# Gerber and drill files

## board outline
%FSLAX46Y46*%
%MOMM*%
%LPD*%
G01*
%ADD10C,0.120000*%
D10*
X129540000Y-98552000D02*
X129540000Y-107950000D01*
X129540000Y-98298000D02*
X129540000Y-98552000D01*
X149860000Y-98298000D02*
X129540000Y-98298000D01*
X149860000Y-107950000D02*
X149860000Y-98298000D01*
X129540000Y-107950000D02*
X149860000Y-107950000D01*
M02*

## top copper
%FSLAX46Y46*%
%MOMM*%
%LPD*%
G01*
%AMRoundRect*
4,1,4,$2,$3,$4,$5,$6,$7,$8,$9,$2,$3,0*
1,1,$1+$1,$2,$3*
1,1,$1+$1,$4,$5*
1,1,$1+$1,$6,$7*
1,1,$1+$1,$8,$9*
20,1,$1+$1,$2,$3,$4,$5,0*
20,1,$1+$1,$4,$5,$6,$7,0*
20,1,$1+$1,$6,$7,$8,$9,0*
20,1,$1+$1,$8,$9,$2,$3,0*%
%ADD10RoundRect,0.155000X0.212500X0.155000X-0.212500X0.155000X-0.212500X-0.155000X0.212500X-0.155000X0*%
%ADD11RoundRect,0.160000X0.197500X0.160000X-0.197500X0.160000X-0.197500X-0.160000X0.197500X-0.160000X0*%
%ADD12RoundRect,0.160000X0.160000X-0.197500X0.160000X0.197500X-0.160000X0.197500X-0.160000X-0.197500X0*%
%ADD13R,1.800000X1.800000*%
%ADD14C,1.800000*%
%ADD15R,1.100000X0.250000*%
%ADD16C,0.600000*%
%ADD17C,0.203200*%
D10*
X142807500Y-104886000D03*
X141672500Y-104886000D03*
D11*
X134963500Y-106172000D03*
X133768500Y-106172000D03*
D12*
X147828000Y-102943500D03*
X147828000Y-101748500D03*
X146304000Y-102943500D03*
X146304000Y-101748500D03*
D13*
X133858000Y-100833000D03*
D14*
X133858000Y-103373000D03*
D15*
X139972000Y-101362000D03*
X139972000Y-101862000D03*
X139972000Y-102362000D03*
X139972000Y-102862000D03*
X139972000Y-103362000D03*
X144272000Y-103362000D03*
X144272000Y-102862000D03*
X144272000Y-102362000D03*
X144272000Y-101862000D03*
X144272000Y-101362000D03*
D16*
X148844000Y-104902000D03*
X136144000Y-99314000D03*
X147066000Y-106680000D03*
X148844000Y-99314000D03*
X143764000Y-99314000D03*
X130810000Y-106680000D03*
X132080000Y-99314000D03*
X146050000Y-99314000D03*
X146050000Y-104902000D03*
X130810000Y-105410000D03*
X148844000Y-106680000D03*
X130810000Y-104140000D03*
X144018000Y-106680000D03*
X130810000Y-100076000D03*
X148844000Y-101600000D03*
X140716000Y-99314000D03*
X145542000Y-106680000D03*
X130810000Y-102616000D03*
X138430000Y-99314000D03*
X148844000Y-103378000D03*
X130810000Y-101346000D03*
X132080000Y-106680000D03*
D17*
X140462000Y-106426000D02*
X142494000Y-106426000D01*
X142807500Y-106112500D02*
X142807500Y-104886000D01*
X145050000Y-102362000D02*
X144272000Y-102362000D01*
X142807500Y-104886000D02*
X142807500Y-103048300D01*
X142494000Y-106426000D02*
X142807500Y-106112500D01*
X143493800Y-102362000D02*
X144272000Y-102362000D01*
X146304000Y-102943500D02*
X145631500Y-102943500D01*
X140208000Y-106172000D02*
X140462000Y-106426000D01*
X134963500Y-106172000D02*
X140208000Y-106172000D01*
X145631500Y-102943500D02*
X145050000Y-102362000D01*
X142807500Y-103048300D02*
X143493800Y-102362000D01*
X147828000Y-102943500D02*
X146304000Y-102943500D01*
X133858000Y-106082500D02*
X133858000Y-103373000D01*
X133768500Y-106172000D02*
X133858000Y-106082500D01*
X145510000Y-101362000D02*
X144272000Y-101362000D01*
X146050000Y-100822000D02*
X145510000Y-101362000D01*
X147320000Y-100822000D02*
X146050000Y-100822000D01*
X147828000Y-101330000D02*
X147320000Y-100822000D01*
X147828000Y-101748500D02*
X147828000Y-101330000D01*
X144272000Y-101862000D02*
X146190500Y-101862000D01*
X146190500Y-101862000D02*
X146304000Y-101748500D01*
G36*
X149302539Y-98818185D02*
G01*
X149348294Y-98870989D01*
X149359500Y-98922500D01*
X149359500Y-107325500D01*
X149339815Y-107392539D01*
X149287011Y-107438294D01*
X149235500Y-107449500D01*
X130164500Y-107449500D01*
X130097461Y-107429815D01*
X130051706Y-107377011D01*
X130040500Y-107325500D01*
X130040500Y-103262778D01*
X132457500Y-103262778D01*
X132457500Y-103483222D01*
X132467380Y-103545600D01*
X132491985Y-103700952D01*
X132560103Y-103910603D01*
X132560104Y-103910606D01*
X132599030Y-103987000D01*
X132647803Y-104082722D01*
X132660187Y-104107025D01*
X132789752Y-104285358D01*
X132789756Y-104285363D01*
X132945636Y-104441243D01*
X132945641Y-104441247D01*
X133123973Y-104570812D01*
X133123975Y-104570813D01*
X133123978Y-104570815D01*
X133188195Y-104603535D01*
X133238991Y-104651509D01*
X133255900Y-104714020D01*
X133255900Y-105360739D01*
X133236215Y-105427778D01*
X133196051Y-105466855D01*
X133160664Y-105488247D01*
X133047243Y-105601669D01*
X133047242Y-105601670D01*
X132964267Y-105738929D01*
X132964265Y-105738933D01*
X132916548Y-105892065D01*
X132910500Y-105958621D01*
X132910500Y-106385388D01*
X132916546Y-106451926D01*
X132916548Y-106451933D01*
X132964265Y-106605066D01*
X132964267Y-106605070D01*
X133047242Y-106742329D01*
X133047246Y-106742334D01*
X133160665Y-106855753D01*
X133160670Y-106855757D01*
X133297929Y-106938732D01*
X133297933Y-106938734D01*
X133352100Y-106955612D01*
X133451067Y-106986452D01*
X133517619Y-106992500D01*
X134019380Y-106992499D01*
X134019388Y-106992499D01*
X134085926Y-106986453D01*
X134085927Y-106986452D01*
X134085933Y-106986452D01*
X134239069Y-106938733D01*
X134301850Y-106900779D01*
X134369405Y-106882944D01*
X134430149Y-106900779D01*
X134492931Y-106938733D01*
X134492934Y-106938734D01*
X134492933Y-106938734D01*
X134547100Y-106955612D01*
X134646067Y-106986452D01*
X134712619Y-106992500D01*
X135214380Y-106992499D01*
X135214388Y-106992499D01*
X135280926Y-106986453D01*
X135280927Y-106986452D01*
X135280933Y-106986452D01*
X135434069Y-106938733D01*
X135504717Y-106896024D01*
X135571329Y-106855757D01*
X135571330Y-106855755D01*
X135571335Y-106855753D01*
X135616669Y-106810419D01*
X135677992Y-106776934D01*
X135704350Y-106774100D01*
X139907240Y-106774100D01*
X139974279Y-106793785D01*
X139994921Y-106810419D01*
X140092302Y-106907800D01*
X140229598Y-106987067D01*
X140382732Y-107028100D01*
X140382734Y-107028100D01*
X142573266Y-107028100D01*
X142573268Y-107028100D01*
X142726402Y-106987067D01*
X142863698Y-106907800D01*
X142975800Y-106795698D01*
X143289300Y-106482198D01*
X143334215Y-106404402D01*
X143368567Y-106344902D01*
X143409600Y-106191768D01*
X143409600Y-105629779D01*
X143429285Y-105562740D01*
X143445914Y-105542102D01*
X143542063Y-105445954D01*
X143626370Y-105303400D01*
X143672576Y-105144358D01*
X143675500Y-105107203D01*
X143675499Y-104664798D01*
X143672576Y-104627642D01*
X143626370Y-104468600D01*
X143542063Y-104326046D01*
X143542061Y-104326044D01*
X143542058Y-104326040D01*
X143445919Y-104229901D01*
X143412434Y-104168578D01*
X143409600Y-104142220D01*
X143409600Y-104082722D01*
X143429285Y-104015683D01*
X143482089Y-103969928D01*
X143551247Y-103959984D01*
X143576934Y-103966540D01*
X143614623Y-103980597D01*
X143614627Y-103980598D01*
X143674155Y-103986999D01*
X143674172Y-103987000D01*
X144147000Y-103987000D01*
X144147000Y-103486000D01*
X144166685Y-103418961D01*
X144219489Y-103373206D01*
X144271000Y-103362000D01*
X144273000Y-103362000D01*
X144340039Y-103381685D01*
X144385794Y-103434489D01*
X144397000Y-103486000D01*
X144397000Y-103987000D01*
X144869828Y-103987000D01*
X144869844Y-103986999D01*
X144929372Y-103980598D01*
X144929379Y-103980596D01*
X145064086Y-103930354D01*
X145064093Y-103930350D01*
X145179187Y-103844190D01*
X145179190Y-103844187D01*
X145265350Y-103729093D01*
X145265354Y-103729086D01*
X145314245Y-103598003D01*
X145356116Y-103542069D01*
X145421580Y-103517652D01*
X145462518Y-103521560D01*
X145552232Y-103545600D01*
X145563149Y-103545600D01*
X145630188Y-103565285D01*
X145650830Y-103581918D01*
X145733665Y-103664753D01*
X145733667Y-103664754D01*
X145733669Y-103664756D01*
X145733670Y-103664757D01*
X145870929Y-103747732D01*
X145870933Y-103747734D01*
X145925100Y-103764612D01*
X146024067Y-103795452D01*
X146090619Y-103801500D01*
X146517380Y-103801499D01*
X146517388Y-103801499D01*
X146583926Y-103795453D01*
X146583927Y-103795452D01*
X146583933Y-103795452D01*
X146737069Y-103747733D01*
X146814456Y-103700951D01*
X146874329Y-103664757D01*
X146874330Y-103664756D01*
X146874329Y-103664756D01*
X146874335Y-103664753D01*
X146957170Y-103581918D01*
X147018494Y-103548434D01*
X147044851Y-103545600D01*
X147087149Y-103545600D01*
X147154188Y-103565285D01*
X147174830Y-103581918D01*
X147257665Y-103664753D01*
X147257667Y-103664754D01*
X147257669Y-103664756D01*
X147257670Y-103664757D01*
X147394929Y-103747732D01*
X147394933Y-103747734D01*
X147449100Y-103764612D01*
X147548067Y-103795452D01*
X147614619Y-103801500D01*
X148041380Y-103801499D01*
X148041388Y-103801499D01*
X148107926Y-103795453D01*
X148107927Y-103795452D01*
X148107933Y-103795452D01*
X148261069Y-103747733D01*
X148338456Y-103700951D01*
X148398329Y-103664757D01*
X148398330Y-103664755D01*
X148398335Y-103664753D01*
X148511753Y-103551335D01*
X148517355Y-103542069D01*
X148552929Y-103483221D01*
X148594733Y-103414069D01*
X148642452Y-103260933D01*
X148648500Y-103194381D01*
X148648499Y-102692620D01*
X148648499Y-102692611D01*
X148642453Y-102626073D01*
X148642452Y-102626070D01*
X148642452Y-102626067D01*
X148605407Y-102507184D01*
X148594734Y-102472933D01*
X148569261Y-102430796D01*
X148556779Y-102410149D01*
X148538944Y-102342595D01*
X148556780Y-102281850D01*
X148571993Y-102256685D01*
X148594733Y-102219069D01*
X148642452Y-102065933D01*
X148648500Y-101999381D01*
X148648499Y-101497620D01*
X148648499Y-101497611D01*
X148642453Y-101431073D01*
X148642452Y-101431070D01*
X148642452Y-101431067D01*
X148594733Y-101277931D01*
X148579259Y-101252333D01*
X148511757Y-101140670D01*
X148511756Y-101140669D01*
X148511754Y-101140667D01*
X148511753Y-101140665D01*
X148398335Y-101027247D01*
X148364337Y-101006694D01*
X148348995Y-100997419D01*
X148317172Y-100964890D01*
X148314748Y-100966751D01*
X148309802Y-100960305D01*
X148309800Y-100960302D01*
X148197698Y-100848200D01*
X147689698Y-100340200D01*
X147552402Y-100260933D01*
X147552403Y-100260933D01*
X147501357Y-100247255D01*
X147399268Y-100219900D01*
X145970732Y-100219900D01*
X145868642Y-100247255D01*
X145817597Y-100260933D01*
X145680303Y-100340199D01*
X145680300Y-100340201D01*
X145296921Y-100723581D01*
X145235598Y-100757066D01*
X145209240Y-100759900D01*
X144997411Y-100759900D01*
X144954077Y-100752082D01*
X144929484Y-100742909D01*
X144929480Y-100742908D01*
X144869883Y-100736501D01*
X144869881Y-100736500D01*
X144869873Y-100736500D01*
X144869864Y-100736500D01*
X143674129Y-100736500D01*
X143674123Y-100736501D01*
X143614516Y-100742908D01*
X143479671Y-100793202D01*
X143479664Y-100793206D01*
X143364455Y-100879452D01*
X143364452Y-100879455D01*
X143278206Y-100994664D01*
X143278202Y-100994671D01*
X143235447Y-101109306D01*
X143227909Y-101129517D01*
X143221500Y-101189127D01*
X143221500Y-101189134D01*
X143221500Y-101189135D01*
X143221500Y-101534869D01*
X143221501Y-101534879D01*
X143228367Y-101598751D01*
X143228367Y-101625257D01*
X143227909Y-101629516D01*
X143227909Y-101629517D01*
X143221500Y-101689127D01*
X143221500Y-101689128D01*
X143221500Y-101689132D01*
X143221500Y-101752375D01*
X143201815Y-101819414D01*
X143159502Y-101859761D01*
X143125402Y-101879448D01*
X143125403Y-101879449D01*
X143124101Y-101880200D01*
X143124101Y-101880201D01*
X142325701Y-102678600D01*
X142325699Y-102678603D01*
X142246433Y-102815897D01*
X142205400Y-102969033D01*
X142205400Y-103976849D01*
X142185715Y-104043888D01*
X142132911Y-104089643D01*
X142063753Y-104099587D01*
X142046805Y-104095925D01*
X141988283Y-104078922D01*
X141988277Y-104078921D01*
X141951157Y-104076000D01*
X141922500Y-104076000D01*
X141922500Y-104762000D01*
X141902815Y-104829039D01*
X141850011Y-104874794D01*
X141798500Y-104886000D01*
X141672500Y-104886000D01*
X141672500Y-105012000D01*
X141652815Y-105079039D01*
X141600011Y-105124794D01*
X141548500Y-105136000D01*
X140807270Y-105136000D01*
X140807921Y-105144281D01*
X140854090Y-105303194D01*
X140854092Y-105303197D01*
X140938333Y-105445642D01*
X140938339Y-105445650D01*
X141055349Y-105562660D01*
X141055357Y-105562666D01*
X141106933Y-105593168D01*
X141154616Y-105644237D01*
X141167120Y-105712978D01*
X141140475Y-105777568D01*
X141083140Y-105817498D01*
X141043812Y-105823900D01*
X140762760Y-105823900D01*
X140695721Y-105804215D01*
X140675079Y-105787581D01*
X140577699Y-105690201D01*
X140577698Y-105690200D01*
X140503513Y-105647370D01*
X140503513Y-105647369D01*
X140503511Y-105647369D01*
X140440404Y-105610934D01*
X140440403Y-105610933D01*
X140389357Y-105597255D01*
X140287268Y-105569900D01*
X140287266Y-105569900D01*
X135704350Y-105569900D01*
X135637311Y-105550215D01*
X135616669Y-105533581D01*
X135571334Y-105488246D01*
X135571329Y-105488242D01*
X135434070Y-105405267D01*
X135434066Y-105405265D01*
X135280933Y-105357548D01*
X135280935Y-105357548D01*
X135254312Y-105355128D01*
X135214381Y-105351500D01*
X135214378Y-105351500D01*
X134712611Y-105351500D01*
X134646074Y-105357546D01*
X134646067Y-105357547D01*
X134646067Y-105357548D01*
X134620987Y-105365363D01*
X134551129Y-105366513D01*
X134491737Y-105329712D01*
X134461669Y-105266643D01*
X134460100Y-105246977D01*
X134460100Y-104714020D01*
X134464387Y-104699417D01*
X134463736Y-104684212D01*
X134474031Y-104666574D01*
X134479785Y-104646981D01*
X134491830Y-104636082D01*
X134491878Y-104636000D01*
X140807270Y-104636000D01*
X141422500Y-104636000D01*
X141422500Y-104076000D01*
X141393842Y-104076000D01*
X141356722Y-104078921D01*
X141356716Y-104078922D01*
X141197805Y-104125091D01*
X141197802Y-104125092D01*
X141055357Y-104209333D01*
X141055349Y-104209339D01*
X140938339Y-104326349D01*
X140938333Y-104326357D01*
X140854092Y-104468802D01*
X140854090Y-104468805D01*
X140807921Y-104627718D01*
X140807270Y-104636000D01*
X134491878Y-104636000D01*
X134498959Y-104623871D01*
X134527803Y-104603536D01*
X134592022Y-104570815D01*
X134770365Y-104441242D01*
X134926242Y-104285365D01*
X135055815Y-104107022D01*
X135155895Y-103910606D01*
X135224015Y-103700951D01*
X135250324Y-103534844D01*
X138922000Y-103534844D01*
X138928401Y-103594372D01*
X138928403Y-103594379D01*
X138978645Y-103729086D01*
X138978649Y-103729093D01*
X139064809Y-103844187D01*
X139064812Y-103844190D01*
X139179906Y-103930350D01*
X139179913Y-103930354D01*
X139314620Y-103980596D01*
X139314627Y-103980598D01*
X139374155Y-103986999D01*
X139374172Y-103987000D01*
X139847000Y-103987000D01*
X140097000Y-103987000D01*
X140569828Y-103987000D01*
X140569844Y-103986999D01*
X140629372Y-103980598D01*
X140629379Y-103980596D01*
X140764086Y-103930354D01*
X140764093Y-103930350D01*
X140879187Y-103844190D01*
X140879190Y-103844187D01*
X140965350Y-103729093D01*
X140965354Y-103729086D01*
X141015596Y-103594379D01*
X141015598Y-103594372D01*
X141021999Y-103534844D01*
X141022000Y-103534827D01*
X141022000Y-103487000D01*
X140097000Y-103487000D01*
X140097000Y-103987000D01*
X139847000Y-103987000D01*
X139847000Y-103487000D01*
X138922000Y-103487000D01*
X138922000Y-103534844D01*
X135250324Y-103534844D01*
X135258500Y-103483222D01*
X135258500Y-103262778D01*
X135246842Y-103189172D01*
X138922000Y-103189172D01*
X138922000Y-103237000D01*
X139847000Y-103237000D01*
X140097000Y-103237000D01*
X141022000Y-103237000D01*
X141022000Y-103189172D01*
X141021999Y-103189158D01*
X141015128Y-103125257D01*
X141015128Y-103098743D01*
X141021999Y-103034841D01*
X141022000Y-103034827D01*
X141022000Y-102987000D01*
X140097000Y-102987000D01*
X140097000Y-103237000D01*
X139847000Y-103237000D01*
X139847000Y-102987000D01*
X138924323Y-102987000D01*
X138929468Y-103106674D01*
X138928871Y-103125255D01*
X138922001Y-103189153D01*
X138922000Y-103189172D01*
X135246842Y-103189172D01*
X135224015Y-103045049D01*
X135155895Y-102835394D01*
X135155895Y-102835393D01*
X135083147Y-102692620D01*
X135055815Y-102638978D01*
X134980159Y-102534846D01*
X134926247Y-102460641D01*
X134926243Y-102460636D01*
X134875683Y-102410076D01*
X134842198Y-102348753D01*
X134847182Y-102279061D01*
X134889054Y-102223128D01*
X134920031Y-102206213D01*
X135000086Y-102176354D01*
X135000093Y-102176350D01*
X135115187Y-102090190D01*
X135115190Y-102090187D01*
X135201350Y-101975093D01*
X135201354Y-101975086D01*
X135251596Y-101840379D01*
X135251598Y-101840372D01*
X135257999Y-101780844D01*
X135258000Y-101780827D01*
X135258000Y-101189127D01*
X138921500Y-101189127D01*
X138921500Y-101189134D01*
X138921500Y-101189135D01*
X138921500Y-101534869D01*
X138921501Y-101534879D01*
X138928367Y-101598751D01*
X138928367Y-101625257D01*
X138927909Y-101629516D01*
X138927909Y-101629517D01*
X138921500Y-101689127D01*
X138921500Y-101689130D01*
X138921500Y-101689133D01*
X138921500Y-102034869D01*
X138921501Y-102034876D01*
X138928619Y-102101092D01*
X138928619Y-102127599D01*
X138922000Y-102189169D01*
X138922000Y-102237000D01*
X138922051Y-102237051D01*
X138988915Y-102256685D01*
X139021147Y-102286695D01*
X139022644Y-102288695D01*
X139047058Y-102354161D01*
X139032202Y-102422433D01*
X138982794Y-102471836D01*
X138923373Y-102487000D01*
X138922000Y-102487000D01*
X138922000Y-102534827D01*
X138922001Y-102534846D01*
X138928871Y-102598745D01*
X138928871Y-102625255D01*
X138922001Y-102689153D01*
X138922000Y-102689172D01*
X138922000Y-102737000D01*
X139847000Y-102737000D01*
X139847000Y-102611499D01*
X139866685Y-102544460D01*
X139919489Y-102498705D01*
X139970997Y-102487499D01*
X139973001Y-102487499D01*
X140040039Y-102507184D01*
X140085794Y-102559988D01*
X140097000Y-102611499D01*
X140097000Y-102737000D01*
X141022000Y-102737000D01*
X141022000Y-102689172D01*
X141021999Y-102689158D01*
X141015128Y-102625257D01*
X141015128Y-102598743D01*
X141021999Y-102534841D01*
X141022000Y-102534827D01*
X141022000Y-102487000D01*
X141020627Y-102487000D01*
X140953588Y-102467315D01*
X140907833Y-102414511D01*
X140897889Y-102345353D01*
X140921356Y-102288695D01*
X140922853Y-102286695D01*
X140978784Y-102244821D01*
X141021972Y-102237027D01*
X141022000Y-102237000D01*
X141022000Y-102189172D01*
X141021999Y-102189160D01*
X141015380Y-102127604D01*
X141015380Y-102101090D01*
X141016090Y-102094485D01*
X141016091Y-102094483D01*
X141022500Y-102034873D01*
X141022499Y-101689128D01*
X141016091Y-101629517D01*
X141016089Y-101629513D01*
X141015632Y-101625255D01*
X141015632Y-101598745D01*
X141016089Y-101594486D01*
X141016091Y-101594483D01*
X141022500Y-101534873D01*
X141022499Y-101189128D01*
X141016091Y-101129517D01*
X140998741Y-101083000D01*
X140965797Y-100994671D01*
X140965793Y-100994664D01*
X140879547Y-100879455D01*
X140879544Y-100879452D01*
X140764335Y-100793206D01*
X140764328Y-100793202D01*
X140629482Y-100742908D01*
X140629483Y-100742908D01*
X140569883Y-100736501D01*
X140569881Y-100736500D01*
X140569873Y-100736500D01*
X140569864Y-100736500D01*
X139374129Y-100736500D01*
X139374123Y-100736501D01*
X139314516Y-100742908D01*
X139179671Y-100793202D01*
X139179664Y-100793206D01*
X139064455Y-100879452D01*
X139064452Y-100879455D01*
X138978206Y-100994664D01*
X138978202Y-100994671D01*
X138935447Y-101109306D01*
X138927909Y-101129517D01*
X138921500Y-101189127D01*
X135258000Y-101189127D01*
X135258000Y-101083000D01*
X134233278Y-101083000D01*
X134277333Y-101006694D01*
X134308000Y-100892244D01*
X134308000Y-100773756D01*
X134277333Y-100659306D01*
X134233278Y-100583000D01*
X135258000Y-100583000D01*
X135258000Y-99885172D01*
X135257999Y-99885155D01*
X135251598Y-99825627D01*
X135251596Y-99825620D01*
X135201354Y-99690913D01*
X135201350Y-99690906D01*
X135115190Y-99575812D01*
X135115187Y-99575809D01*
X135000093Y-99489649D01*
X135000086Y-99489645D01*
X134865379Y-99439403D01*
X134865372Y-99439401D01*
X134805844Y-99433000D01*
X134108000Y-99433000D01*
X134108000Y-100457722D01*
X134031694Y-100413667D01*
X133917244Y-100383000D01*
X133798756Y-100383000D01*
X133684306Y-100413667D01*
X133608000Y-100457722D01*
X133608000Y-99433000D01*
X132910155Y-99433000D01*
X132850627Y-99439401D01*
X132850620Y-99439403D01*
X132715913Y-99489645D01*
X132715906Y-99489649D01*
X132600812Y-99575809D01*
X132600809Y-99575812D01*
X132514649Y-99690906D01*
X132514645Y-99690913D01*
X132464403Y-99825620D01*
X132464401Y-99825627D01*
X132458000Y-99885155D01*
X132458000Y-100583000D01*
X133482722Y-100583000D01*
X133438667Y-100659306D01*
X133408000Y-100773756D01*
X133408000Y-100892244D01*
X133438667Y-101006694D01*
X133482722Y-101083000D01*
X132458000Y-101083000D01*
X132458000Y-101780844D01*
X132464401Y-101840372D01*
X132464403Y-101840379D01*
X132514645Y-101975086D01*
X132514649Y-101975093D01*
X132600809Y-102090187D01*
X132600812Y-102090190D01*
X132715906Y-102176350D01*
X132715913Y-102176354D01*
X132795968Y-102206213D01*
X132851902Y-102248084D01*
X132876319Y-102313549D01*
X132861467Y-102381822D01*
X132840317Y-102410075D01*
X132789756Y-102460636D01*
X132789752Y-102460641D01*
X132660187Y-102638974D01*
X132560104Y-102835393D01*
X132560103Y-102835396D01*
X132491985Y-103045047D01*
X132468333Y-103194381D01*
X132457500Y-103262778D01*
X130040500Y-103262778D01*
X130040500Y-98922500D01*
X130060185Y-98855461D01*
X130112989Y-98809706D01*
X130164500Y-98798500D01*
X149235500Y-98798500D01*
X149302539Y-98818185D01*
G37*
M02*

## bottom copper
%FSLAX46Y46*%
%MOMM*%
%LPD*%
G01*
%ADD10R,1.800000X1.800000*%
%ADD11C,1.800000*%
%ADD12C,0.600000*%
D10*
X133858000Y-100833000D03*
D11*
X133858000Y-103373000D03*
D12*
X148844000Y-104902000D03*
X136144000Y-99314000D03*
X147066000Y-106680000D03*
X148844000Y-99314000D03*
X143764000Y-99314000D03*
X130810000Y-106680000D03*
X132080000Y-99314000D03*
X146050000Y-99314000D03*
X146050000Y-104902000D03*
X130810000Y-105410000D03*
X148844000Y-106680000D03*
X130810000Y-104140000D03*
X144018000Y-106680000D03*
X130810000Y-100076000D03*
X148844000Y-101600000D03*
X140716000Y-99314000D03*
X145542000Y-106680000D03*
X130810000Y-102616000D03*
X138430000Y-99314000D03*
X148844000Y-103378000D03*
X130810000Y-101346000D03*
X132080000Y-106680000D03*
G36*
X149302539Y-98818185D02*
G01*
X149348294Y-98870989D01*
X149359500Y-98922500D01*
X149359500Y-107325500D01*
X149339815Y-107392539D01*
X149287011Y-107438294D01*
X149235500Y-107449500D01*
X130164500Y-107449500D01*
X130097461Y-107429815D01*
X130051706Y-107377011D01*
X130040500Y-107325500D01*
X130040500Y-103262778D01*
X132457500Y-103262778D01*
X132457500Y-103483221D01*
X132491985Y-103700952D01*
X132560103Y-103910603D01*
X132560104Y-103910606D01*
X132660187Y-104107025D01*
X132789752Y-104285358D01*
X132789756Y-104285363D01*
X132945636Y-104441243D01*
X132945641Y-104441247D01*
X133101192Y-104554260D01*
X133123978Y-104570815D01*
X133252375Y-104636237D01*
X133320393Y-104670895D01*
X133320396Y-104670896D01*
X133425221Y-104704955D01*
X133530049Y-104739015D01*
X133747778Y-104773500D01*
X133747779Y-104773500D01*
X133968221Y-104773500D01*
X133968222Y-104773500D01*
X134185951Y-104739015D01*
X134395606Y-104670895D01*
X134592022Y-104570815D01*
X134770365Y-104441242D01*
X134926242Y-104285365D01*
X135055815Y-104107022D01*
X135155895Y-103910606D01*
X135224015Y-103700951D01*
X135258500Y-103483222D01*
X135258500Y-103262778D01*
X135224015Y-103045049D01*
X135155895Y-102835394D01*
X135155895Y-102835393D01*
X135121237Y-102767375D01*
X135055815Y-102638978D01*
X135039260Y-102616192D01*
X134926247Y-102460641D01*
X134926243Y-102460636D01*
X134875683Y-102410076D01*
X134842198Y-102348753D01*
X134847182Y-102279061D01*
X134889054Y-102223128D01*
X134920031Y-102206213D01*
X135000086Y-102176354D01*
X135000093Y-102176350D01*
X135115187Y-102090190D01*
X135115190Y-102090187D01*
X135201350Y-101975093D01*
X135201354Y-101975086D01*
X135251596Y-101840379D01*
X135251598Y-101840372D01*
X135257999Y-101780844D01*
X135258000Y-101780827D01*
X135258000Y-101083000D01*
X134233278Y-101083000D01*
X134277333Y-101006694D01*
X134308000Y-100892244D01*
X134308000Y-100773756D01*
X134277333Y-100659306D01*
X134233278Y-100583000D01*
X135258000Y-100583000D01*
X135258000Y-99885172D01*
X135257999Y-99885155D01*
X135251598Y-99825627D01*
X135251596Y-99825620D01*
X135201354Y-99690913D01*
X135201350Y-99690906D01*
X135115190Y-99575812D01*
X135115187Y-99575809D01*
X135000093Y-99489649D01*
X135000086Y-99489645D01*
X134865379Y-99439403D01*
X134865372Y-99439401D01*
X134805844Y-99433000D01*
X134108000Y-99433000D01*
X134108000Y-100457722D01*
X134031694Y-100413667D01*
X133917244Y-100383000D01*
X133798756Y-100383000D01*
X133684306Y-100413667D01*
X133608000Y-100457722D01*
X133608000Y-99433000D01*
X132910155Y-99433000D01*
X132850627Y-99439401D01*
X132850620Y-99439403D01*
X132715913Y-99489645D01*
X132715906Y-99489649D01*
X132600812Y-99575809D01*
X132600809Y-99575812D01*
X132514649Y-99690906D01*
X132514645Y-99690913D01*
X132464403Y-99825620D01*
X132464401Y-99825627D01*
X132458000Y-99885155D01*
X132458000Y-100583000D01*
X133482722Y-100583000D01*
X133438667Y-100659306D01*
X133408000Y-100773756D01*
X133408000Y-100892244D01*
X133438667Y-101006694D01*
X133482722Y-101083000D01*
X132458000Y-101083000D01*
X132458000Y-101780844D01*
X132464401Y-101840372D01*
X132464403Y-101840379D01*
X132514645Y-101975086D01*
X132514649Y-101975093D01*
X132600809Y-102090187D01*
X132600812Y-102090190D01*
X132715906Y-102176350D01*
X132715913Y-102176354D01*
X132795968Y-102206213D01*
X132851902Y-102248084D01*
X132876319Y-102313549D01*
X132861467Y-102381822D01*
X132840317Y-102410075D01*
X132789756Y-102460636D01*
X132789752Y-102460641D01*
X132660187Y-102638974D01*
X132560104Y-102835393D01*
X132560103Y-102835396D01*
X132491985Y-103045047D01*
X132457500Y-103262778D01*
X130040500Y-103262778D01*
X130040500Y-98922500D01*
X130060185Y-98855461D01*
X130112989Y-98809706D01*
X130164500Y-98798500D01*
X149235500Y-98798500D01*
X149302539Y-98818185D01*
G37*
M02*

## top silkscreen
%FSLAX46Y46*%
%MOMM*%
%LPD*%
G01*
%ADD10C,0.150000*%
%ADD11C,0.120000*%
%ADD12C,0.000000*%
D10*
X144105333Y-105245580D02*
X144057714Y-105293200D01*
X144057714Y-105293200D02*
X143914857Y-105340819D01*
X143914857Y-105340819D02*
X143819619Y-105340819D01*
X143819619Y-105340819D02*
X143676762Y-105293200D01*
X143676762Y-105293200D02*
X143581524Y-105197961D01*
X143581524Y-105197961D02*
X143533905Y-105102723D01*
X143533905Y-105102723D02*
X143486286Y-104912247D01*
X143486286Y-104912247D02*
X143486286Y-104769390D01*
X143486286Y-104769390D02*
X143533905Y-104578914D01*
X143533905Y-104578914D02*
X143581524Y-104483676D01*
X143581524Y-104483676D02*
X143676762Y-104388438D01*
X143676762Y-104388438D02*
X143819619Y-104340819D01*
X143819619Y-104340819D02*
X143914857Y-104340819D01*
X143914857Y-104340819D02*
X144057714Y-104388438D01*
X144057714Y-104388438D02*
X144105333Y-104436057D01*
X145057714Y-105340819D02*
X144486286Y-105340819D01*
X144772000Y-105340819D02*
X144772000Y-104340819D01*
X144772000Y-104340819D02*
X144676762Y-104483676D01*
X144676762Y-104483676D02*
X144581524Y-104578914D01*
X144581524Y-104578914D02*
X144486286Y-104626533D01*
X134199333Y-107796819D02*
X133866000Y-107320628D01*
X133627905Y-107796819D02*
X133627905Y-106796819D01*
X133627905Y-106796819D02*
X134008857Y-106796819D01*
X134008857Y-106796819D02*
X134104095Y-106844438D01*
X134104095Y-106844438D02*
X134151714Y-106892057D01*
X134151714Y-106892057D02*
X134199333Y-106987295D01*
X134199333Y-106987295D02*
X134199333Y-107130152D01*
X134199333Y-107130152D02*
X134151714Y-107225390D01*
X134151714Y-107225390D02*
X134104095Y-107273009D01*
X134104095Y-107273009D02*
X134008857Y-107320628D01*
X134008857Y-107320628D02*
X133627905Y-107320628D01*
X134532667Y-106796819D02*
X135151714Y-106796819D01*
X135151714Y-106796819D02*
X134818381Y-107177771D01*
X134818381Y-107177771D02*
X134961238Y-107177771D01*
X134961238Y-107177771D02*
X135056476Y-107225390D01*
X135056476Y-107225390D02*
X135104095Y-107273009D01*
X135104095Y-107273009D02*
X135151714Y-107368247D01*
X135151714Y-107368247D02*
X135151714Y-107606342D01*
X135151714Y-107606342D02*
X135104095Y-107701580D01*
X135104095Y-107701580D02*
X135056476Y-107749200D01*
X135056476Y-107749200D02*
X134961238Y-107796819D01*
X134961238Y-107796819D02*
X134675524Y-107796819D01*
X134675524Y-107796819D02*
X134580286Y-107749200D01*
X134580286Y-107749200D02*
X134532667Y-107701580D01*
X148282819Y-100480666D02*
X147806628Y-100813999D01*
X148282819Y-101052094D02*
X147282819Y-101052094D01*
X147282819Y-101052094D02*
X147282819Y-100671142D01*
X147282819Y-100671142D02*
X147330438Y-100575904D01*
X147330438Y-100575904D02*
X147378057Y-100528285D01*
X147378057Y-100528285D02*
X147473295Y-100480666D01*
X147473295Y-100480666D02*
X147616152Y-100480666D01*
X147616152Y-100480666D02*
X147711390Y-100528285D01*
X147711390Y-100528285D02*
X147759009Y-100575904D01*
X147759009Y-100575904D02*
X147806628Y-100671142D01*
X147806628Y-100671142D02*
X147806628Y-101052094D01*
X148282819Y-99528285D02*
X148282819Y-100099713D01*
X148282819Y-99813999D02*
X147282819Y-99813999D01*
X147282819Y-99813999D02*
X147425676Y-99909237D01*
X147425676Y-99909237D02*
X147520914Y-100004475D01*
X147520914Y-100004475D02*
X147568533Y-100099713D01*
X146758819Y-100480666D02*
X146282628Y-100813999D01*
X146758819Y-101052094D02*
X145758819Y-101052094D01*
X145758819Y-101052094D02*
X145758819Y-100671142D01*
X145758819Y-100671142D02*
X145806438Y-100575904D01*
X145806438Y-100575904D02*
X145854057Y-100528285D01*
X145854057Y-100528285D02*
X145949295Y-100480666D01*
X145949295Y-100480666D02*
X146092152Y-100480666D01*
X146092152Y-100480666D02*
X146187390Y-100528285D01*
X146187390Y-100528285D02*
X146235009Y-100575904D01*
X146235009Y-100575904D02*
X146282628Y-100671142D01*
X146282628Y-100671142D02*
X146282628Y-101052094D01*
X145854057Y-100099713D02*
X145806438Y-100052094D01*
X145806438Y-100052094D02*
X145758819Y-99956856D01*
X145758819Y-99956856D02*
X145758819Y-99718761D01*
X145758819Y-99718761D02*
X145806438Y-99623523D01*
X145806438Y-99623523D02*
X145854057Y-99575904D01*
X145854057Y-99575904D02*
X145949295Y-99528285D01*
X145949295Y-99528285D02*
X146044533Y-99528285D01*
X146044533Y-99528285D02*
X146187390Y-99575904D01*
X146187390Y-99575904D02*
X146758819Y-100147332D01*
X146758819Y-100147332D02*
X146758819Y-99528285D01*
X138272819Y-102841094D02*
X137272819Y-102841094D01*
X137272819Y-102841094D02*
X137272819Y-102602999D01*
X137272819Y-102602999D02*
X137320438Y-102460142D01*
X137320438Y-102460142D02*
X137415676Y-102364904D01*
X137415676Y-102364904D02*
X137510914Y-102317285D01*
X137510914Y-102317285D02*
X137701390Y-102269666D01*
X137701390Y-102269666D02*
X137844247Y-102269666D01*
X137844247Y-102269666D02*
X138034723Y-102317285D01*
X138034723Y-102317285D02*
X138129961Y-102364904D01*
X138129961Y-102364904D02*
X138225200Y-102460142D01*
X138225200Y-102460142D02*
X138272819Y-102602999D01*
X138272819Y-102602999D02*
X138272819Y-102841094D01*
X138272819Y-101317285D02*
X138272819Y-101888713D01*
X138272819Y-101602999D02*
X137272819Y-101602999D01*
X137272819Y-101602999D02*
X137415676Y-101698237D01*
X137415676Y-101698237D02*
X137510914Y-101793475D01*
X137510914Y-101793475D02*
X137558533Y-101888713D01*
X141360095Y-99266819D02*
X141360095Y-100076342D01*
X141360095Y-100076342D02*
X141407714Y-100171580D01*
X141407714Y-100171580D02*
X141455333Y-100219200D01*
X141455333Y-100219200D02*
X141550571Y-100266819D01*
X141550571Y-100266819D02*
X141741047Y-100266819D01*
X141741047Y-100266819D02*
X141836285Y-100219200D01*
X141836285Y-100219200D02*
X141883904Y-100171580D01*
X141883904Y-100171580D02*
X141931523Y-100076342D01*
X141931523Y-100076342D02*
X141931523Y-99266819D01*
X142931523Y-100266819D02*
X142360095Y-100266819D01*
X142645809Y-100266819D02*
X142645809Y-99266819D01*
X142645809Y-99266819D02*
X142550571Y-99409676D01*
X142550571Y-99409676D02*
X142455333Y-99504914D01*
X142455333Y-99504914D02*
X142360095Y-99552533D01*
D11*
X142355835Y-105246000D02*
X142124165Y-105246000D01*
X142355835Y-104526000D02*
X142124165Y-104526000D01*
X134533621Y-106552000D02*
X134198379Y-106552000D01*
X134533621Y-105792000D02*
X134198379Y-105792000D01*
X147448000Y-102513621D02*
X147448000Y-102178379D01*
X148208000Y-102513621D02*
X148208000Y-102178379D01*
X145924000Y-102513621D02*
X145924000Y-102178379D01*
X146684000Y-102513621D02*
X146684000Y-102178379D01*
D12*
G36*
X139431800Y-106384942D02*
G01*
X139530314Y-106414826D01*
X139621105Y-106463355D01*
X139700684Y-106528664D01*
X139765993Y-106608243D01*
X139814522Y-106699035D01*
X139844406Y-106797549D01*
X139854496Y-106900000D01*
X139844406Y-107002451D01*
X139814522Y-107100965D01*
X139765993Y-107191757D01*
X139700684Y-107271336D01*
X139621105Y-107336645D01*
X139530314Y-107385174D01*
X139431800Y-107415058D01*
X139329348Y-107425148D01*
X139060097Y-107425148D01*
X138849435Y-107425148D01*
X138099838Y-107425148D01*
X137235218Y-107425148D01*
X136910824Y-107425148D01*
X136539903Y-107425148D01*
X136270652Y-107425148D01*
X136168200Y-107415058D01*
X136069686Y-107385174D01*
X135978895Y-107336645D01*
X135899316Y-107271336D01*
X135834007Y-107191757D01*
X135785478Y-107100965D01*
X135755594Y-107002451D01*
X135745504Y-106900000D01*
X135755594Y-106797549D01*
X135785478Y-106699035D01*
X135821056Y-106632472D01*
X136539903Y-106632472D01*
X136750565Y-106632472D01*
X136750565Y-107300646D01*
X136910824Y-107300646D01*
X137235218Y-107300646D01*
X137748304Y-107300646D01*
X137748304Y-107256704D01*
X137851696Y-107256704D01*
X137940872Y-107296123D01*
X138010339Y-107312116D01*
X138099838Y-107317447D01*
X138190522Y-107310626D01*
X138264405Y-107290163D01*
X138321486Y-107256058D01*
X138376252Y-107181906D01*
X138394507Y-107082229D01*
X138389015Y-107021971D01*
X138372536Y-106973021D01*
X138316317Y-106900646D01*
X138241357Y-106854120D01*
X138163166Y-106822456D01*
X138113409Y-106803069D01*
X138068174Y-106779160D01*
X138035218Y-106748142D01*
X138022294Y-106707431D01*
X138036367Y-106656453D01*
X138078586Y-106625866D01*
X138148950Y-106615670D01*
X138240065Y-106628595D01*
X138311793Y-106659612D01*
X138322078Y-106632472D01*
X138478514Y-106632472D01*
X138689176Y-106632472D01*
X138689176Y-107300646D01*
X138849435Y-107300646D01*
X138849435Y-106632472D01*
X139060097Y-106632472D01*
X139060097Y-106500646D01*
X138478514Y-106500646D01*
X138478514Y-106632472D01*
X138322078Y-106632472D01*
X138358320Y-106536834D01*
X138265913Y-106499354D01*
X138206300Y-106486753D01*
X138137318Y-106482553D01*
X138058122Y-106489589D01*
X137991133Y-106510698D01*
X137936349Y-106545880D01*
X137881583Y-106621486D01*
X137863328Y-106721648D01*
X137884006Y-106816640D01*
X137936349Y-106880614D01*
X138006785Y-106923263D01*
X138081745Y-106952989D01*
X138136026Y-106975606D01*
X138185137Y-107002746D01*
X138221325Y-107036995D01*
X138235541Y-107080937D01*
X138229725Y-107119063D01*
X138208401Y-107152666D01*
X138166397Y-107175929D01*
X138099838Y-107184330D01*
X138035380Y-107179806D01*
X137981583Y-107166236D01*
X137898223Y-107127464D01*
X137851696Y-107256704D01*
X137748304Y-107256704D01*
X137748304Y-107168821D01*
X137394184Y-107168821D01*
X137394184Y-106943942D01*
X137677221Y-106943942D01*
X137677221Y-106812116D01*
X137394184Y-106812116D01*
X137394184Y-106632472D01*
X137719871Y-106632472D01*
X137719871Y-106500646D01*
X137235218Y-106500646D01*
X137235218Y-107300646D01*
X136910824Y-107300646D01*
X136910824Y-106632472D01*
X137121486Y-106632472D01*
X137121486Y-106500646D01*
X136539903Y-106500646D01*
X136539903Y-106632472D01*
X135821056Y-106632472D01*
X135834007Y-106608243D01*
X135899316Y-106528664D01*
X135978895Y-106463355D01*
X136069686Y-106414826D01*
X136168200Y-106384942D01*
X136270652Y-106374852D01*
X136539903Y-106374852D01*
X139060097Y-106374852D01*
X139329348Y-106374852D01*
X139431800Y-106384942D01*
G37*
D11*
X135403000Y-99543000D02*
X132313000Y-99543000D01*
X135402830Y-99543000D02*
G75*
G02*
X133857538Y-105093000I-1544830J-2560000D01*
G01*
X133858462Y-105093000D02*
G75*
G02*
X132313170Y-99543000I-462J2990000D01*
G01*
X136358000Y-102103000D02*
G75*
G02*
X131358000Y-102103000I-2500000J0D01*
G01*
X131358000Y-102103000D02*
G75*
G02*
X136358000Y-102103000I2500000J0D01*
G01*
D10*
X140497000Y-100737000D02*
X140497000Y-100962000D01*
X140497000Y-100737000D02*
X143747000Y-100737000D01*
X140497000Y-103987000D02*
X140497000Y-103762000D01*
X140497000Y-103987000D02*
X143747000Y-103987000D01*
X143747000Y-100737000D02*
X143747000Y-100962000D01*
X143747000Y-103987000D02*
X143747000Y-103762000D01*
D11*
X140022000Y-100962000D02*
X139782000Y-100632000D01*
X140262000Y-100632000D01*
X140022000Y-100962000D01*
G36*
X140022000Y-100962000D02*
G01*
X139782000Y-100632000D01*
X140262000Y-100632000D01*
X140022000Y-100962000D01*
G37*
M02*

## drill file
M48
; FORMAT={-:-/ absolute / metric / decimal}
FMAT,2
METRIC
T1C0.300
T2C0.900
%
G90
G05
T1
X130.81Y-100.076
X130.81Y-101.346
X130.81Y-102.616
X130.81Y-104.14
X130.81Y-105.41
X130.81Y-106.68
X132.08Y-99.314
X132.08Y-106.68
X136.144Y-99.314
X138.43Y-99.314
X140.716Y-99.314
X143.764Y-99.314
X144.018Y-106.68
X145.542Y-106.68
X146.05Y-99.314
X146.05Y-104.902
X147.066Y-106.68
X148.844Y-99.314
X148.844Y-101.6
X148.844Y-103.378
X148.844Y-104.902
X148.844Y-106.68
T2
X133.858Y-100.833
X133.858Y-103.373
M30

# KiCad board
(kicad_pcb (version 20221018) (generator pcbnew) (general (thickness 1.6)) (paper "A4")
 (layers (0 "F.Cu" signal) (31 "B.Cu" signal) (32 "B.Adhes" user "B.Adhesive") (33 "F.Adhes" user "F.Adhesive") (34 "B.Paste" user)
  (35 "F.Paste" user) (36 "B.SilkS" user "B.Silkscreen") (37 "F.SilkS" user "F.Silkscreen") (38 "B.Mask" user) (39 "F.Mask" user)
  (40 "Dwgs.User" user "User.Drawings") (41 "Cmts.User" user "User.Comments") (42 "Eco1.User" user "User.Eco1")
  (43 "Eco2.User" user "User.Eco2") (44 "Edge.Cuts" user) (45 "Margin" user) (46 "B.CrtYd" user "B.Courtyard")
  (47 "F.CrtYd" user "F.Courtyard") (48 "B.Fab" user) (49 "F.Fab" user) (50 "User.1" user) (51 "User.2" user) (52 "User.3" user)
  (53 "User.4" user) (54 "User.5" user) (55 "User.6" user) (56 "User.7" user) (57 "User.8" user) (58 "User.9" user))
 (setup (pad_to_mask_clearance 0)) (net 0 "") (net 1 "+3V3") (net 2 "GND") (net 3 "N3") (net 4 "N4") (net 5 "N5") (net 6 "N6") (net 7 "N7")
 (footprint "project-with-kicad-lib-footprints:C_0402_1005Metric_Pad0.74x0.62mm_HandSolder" (layer "F.Cu") (at 142.24 104.886 180)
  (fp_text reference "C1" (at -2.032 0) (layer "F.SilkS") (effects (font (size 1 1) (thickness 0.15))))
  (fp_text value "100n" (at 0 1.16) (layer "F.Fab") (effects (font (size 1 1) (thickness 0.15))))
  (fp_line (start -0.115835 -0.36) (end 0.115835 -0.36) (layer "F.SilkS") (stroke (width 0.12) (type solid)))
  (fp_line (start -0.115835 0.36) (end 0.115835 0.36) (layer "F.SilkS") (stroke (width 0.12) (type solid)))
  (pad "1" smd roundrect (at -0.5675 0 180) (size 0.735 0.62) (layers "F.Cu" "F.Paste" "F.Mask") (roundrect_rratio 0.25) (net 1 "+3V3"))
  (pad "2" smd roundrect (at 0.5675 0 180) (size 0.735 0.62) (layers "F.Cu" "F.Paste" "F.Mask") (roundrect_rratio 0.25) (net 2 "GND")))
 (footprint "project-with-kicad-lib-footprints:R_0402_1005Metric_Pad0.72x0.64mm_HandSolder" (layer "F.Cu") (at 134.366 106.172 180)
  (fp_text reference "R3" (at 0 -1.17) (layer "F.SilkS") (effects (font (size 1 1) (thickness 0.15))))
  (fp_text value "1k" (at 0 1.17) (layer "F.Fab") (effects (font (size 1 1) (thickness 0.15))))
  (fp_line (start -0.167621 -0.38) (end 0.167621 -0.38) (layer "F.SilkS") (stroke (width 0.12) (type solid)))
  (fp_line (start -0.167621 0.38) (end 0.167621 0.38) (layer "F.SilkS") (stroke (width 0.12) (type solid)))
  (pad "1" smd roundrect (at -0.5975 0 180) (size 0.715 0.64) (layers "F.Cu" "F.Paste" "F.Mask") (roundrect_rratio 0.25) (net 1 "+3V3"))
  (pad "2" smd roundrect (at 0.5975 0 180) (size 0.715 0.64) (layers "F.Cu" "F.Paste" "F.Mask") (roundrect_rratio 0.25) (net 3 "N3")))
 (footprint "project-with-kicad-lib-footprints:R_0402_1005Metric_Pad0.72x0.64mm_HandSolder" (layer "F.Cu") (at 147.828 102.346 90)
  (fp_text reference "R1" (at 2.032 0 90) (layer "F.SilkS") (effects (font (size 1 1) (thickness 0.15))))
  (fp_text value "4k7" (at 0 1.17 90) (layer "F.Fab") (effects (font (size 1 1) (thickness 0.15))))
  (fp_line (start -0.167621 -0.38) (end 0.167621 -0.38) (layer "F.SilkS") (stroke (width 0.12) (type solid)))
  (fp_line (start -0.167621 0.38) (end 0.167621 0.38) (layer "F.SilkS") (stroke (width 0.12) (type solid)))
  (pad "1" smd roundrect (at -0.5975 0 90) (size 0.715 0.64) (layers "F.Cu" "F.Paste" "F.Mask") (roundrect_rratio 0.25) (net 1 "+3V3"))
  (pad "2" smd roundrect (at 0.5975 0 90) (size 0.715 0.64) (layers "F.Cu" "F.Paste" "F.Mask") (roundrect_rratio 0.25) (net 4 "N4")))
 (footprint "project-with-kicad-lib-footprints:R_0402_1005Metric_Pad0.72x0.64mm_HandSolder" (layer "F.Cu") (at 146.304 102.346 90)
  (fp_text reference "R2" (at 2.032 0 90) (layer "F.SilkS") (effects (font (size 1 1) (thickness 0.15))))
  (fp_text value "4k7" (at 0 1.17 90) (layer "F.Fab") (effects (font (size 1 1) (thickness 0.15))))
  (fp_line (start -0.167621 -0.38) (end 0.167621 -0.38) (layer "F.SilkS") (stroke (width 0.12) (type solid)))
  (fp_line (start -0.167621 0.38) (end 0.167621 0.38) (layer "F.SilkS") (stroke (width 0.12) (type solid)))
  (pad "1" smd roundrect (at -0.5975 0 90) (size 0.715 0.64) (layers "F.Cu" "F.Paste" "F.Mask") (roundrect_rratio 0.25) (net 1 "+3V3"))
  (pad "2" smd roundrect (at 0.5975 0 90) (size 0.715 0.64) (layers "F.Cu" "F.Paste" "F.Mask") (roundrect_rratio 0.25) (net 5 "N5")))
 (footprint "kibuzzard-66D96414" (layer "F.Cu") (at 137.8 106.9)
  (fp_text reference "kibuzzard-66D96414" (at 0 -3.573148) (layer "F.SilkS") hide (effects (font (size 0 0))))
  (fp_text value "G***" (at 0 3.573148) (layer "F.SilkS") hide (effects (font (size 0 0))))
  (fp_poly
   (pts (xy -1.260097 -0.525148) (xy -1.529348 -0.525148) (xy -1.6318 -0.515058) (xy -1.730314 -0.485174) (xy -1.821105 -0.436645)
    (xy -1.900684 -0.371336) (xy -1.965993 -0.291757) (xy -2.014522 -0.200965) (xy -2.044406 -0.102451) (xy -2.054496 0)
    (xy -2.044406 0.102451) (xy -2.014522 0.200965) (xy -1.965993 0.291757) (xy -1.900684 0.371336) (xy -1.821105 0.436645)
    (xy -1.730314 0.485174) (xy -1.6318 0.515058) (xy -1.529348 0.525148) (xy -1.260097 0.525148) (xy -0.889176 0.525148)
    (xy -0.889176 0.400646) (xy -1.049435 0.400646) (xy -1.049435 -0.267528) (xy -1.260097 -0.267528) (xy -1.260097 -0.399354)
    (xy -0.678514 -0.399354) (xy -0.678514 -0.267528) (xy -0.889176 -0.267528) (xy -0.889176 0.400646) (xy -0.889176 0.525148)
    (xy -0.564782 0.525148) (xy -0.564782 0.400646) (xy -0.564782 -0.399354) (xy -0.080129 -0.399354) (xy -0.080129 -0.267528)
    (xy -0.405816 -0.267528) (xy -0.405816 -0.087884) (xy -0.122779 -0.087884) (xy -0.122779 0.043942) (xy -0.405816 0.043942)
    (xy -0.405816 0.268821) (xy -0.051696 0.268821) (xy -0.051696 0.400646) (xy -0.564782 0.400646) (xy -0.564782 0.525148)
    (xy 0.299838 0.525148) (xy 0.299838 0.417447) (xy 0.210339 0.412116) (xy 0.140872 0.396123) (xy 0.051696 0.356704)
    (xy 0.098223 0.227464) (xy 0.181583 0.266236) (xy 0.23538 0.279806) (xy 0.299838 0.28433) (xy 0.366397 0.275929) (xy 0.408401 0.252666)
    (xy 0.429725 0.219063) (xy 0.435541 0.180937) (xy 0.421325 0.136995) (xy 0.385137 0.102746) (xy 0.336026 0.075606)
    (xy 0.281745 0.052989) (xy 0.206785 0.023263) (xy 0.136349 -0.019386) (xy 0.084006 -0.08336) (xy 0.063328 -0.178352)
    (xy 0.081583 -0.278514) (xy 0.136349 -0.35412) (xy 0.191133 -0.389302) (xy 0.258122 -0.410411) (xy 0.337318 -0.417447)
    (xy 0.4063 -0.413247) (xy 0.465913 -0.400646) (xy 0.55832 -0.363166) (xy 0.511793 -0.240388) (xy 0.440065 -0.271405)
    (xy 0.34895 -0.28433) (xy 0.278586 -0.274134) (xy 0.236367 -0.243547) (xy 0.222294 -0.192569) (xy 0.235218 -0.151858)
    (xy 0.268174 -0.12084) (xy 0.313409 -0.096931) (xy 0.363166 -0.077544) (xy 0.441357 -0.04588) (xy 0.516317 0.000646)
    (xy 0.572536 0.073021) (xy 0.589015 0.121971) (xy 0.594507 0.182229) (xy 0.576252 0.281906) (xy 0.521486 0.356058)
    (xy 0.464405 0.390163) (xy 0.390522 0.410626) (xy 0.299838 0.417447) (xy 0.299838 0.525148) (xy 1.049435 0.525148)
    (xy 1.049435 0.400646) (xy 0.889176 0.400646) (xy 0.889176 -0.267528) (xy 0.678514 -0.267528) (xy 0.678514 -0.399354)
    (xy 1.260097 -0.399354) (xy 1.260097 -0.267528) (xy 1.049435 -0.267528) (xy 1.049435 0.400646) (xy 1.049435 0.525148)
    (xy 1.260097 0.525148) (xy 1.529348 0.525148) (xy 1.6318 0.515058) (xy 1.730314 0.485174) (xy 1.821105 0.436645) (xy 1.900684 0.371336)
    (xy 1.965993 0.291757) (xy 2.014522 0.200965) (xy 2.044406 0.102451) (xy 2.054496 0) (xy 2.044406 -0.102451) (xy 2.014522 -0.200965)
    (xy 1.965993 -0.291757) (xy 1.900684 -0.371336) (xy 1.821105 -0.436645) (xy 1.730314 -0.485174) (xy 1.6318 -0.515058)
    (xy 1.529348 -0.525148) (xy 1.260097 -0.525148) (xy -1.260097 -0.525148))
   (layer "F.SilkS") (stroke (width 0) (type solid)) (fill solid)))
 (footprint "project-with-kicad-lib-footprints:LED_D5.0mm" (layer "F.Cu") (at 133.858 100.833 -90)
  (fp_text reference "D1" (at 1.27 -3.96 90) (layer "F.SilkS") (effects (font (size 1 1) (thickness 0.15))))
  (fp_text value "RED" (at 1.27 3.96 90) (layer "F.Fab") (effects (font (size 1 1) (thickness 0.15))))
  (fp_line (start -1.29 -1.545) (end -1.29 1.545) (layer "F.SilkS") (stroke (width 0.12) (type solid)))
  (fp_arc (start -1.29 -1.54483) (mid 2.072002 -2.880433) (end 4.26 0.000462) (layer "F.SilkS") (stroke (width 0.12) (type solid)))
  (fp_arc (start 4.26 -0.000462) (mid 2.072002 2.880433) (end -1.29 1.54483) (layer "F.SilkS") (stroke (width 0.12) (type solid)))
  (fp_circle (center 1.27 0) (end 3.77 0) (layer "F.SilkS") (stroke (width 0.12) (type solid)) (fill none))
  (pad "1" thru_hole rect (at 0 0 270) (size 1.8 1.8) (drill 0.9) (layers *.Cu *.Mask) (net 2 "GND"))
  (pad "2" thru_hole circle (at 2.54 0 270) (size 1.8 1.8) (drill 0.9) (layers *.Cu *.Mask) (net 3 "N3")))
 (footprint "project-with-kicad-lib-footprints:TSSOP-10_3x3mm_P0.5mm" (layer "F.Cu") (at 142.122 102.362)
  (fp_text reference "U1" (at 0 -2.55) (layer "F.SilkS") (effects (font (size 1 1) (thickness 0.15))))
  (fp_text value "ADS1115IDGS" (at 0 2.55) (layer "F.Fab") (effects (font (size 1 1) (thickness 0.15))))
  (fp_line (start -1.625 -1.625) (end -1.625 -1.4) (layer "F.SilkS") (stroke (width 0.15) (type solid)))
  (fp_line (start -1.625 -1.625) (end 1.625 -1.625) (layer "F.SilkS") (stroke (width 0.15) (type solid)))
  (fp_line (start -1.625 1.625) (end -1.625 1.4) (layer "F.SilkS") (stroke (width 0.15) (type solid)))
  (fp_line (start -1.625 1.625) (end 1.625 1.625) (layer "F.SilkS") (stroke (width 0.15) (type solid)))
  (fp_line (start 1.625 -1.625) (end 1.625 -1.4) (layer "F.SilkS") (stroke (width 0.15) (type solid)))
  (fp_line (start 1.625 1.625) (end 1.625 1.4) (layer "F.SilkS") (stroke (width 0.15) (type solid)))
  (fp_poly
   (pts (xy -2.1 -1.4) (xy -2.34 -1.73) (xy -1.86 -1.73) (xy -2.1 -1.4)) (layer "F.SilkS") (stroke (width 0.12) (type solid)) (fill solid))
  (pad "1" smd rect (at -2.15 -1) (size 1.1 0.25) (layers "F.Cu" "F.Paste" "F.Mask") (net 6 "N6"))
  (pad "2" smd rect (at -2.15 -0.5) (size 1.1 0.25) (layers "F.Cu" "F.Paste" "F.Mask") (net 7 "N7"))
  (pad "3" smd rect (at -2.15 0) (size 1.1 0.25) (layers "F.Cu" "F.Paste" "F.Mask") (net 2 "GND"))
  (pad "4" smd rect (at -2.15 0.5) (size 1.1 0.25) (layers "F.Cu" "F.Paste" "F.Mask") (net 2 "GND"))
  (pad "5" smd rect (at -2.15 1) (size 1.1 0.25) (layers "F.Cu" "F.Paste" "F.Mask") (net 2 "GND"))
  (pad "6" smd rect (at 2.15 1) (size 1.1 0.25) (layers "F.Cu" "F.Paste" "F.Mask") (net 2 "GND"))
  (pad "7" smd rect (at 2.15 0.5) (size 1.1 0.25) (layers "F.Cu" "F.Paste" "F.Mask") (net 2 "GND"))
  (pad "8" smd rect (at 2.15 0) (size 1.1 0.25) (layers "F.Cu" "F.Paste" "F.Mask") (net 1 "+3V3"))
  (pad "9" smd rect (at 2.15 -0.5) (size 1.1 0.25) (layers "F.Cu" "F.Paste" "F.Mask") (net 5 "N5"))
  (pad "10" smd rect (at 2.15 -1) (size 1.1 0.25) (layers "F.Cu" "F.Paste" "F.Mask") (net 4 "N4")))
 (gr_line (start 129.54 98.552) (end 129.54 107.95) (layer "Edge.Cuts") (width 0.12))
 (gr_line (start 129.54 98.298) (end 129.54 98.552) (layer "Edge.Cuts") (width 0.12))
 (gr_line (start 149.86 98.298) (end 129.54 98.298) (layer "Edge.Cuts") (width 0.12))
 (gr_line (start 149.86 107.95) (end 149.86 98.298) (layer "Edge.Cuts") (width 0.12))
 (gr_line (start 129.54 107.95) (end 149.86 107.95) (layer "Edge.Cuts") (width 0.12))
 (segment (start 140.462 106.426) (end 142.494 106.426) (width 0.2032) (layer "F.Cu") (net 1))
 (segment (start 142.8075 106.1125) (end 142.8075 104.886) (width 0.2032) (layer "F.Cu") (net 1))
 (segment (start 145.05 102.362) (end 144.272 102.362) (width 0.2032) (layer "F.Cu") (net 1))
 (segment (start 142.8075 104.886) (end 142.8075 103.0483) (width 0.2032) (layer "F.Cu") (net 1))
 (segment (start 142.494 106.426) (end 142.8075 106.1125) (width 0.2032) (layer "F.Cu") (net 1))
 (segment (start 143.4938 102.362) (end 144.272 102.362) (width 0.2032) (layer "F.Cu") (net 1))
 (segment (start 146.304 102.9435) (end 145.6315 102.9435) (width 0.2032) (layer "F.Cu") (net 1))
 (segment (start 140.208 106.172) (end 140.462 106.426) (width 0.2032) (layer "F.Cu") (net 1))
 (segment (start 134.9635 106.172) (end 140.208 106.172) (width 0.2032) (layer "F.Cu") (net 1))
 (segment (start 145.6315 102.9435) (end 145.05 102.362) (width 0.2032) (layer "F.Cu") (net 1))
 (segment (start 142.8075 103.0483) (end 143.4938 102.362) (width 0.2032) (layer "F.Cu") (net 1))
 (segment (start 147.828 102.9435) (end 146.304 102.9435) (width 0.2032) (layer "F.Cu") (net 1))
 (via (at 148.844 104.902) (size 0.6) (drill 0.3) (layers "F.Cu" "B.Cu") (free) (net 2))
 (via (at 136.144 99.314) (size 0.6) (drill 0.3) (layers "F.Cu" "B.Cu") (free) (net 2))
 (via (at 147.066 106.68) (size 0.6) (drill 0.3) (layers "F.Cu" "B.Cu") (free) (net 2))
 (via (at 148.844 99.314) (size 0.6) (drill 0.3) (layers "F.Cu" "B.Cu") (free) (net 2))
 (via (at 143.764 99.314) (size 0.6) (drill 0.3) (layers "F.Cu" "B.Cu") (free) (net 2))
 (via (at 130.81 106.68) (size 0.6) (drill 0.3) (layers "F.Cu" "B.Cu") (free) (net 2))
 (via (at 132.08 99.314) (size 0.6) (drill 0.3) (layers "F.Cu" "B.Cu") (free) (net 2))
 (via (at 146.05 99.314) (size 0.6) (drill 0.3) (layers "F.Cu" "B.Cu") (free) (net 2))
 (via (at 146.05 104.902) (size 0.6) (drill 0.3) (layers "F.Cu" "B.Cu") (free) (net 2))
 (via (at 130.81 105.41) (size 0.6) (drill 0.3) (layers "F.Cu" "B.Cu") (free) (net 2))
 (via (at 148.844 106.68) (size 0.6) (drill 0.3) (layers "F.Cu" "B.Cu") (free) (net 2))
 (via (at 130.81 104.14) (size 0.6) (drill 0.3) (layers "F.Cu" "B.Cu") (free) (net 2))
 (via (at 144.018 106.68) (size 0.6) (drill 0.3) (layers "F.Cu" "B.Cu") (free) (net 2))
 (via (at 130.81 100.076) (size 0.6) (drill 0.3) (layers "F.Cu" "B.Cu") (free) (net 2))
 (via (at 148.844 101.6) (size 0.6) (drill 0.3) (layers "F.Cu" "B.Cu") (free) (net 2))
 (via (at 140.716 99.314) (size 0.6) (drill 0.3) (layers "F.Cu" "B.Cu") (free) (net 2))
 (via (at 145.542 106.68) (size 0.6) (drill 0.3) (layers "F.Cu" "B.Cu") (free) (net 2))
 (via (at 130.81 102.616) (size 0.6) (drill 0.3) (layers "F.Cu" "B.Cu") (free) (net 2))
 (via (at 138.43 99.314) (size 0.6) (drill 0.3) (layers "F.Cu" "B.Cu") (free) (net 2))
 (via (at 148.844 103.378) (size 0.6) (drill 0.3) (layers "F.Cu" "B.Cu") (free) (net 2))
 (via (at 130.81 101.346) (size 0.6) (drill 0.3) (layers "F.Cu" "B.Cu") (free) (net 2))
 (via (at 132.08 106.68) (size 0.6) (drill 0.3) (layers "F.Cu" "B.Cu") (free) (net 2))
 (segment (start 133.858 106.0825) (end 133.858 103.373) (width 0.2032) (layer "F.Cu") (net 3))
 (segment (start 133.7685 106.172) (end 133.858 106.0825) (width 0.2032) (layer "F.Cu") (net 3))
 (segment (start 145.51 101.362) (end 144.272 101.362) (width 0.2032) (layer "F.Cu") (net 4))
 (segment (start 146.05 100.822) (end 145.51 101.362) (width 0.2032) (layer "F.Cu") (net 4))
 (segment (start 147.32 100.822) (end 146.05 100.822) (width 0.2032) (layer "F.Cu") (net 4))
 (segment (start 147.828 101.33) (end 147.32 100.822) (width 0.2032) (layer "F.Cu") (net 4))
 (segment (start 147.828 101.7485) (end 147.828 101.33) (width 0.2032) (layer "F.Cu") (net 4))
 (segment (start 144.272 101.862) (end 146.1905 101.862) (width 0.2032) (layer "F.Cu") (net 5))
 (segment (start 146.1905 101.862) (end 146.304 101.7485) (width 0.2032) (layer "F.Cu") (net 5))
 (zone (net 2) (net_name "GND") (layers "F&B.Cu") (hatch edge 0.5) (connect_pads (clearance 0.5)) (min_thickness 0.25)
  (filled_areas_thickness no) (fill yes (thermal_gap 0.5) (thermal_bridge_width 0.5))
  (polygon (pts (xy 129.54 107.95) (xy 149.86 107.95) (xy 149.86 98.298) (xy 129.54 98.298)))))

